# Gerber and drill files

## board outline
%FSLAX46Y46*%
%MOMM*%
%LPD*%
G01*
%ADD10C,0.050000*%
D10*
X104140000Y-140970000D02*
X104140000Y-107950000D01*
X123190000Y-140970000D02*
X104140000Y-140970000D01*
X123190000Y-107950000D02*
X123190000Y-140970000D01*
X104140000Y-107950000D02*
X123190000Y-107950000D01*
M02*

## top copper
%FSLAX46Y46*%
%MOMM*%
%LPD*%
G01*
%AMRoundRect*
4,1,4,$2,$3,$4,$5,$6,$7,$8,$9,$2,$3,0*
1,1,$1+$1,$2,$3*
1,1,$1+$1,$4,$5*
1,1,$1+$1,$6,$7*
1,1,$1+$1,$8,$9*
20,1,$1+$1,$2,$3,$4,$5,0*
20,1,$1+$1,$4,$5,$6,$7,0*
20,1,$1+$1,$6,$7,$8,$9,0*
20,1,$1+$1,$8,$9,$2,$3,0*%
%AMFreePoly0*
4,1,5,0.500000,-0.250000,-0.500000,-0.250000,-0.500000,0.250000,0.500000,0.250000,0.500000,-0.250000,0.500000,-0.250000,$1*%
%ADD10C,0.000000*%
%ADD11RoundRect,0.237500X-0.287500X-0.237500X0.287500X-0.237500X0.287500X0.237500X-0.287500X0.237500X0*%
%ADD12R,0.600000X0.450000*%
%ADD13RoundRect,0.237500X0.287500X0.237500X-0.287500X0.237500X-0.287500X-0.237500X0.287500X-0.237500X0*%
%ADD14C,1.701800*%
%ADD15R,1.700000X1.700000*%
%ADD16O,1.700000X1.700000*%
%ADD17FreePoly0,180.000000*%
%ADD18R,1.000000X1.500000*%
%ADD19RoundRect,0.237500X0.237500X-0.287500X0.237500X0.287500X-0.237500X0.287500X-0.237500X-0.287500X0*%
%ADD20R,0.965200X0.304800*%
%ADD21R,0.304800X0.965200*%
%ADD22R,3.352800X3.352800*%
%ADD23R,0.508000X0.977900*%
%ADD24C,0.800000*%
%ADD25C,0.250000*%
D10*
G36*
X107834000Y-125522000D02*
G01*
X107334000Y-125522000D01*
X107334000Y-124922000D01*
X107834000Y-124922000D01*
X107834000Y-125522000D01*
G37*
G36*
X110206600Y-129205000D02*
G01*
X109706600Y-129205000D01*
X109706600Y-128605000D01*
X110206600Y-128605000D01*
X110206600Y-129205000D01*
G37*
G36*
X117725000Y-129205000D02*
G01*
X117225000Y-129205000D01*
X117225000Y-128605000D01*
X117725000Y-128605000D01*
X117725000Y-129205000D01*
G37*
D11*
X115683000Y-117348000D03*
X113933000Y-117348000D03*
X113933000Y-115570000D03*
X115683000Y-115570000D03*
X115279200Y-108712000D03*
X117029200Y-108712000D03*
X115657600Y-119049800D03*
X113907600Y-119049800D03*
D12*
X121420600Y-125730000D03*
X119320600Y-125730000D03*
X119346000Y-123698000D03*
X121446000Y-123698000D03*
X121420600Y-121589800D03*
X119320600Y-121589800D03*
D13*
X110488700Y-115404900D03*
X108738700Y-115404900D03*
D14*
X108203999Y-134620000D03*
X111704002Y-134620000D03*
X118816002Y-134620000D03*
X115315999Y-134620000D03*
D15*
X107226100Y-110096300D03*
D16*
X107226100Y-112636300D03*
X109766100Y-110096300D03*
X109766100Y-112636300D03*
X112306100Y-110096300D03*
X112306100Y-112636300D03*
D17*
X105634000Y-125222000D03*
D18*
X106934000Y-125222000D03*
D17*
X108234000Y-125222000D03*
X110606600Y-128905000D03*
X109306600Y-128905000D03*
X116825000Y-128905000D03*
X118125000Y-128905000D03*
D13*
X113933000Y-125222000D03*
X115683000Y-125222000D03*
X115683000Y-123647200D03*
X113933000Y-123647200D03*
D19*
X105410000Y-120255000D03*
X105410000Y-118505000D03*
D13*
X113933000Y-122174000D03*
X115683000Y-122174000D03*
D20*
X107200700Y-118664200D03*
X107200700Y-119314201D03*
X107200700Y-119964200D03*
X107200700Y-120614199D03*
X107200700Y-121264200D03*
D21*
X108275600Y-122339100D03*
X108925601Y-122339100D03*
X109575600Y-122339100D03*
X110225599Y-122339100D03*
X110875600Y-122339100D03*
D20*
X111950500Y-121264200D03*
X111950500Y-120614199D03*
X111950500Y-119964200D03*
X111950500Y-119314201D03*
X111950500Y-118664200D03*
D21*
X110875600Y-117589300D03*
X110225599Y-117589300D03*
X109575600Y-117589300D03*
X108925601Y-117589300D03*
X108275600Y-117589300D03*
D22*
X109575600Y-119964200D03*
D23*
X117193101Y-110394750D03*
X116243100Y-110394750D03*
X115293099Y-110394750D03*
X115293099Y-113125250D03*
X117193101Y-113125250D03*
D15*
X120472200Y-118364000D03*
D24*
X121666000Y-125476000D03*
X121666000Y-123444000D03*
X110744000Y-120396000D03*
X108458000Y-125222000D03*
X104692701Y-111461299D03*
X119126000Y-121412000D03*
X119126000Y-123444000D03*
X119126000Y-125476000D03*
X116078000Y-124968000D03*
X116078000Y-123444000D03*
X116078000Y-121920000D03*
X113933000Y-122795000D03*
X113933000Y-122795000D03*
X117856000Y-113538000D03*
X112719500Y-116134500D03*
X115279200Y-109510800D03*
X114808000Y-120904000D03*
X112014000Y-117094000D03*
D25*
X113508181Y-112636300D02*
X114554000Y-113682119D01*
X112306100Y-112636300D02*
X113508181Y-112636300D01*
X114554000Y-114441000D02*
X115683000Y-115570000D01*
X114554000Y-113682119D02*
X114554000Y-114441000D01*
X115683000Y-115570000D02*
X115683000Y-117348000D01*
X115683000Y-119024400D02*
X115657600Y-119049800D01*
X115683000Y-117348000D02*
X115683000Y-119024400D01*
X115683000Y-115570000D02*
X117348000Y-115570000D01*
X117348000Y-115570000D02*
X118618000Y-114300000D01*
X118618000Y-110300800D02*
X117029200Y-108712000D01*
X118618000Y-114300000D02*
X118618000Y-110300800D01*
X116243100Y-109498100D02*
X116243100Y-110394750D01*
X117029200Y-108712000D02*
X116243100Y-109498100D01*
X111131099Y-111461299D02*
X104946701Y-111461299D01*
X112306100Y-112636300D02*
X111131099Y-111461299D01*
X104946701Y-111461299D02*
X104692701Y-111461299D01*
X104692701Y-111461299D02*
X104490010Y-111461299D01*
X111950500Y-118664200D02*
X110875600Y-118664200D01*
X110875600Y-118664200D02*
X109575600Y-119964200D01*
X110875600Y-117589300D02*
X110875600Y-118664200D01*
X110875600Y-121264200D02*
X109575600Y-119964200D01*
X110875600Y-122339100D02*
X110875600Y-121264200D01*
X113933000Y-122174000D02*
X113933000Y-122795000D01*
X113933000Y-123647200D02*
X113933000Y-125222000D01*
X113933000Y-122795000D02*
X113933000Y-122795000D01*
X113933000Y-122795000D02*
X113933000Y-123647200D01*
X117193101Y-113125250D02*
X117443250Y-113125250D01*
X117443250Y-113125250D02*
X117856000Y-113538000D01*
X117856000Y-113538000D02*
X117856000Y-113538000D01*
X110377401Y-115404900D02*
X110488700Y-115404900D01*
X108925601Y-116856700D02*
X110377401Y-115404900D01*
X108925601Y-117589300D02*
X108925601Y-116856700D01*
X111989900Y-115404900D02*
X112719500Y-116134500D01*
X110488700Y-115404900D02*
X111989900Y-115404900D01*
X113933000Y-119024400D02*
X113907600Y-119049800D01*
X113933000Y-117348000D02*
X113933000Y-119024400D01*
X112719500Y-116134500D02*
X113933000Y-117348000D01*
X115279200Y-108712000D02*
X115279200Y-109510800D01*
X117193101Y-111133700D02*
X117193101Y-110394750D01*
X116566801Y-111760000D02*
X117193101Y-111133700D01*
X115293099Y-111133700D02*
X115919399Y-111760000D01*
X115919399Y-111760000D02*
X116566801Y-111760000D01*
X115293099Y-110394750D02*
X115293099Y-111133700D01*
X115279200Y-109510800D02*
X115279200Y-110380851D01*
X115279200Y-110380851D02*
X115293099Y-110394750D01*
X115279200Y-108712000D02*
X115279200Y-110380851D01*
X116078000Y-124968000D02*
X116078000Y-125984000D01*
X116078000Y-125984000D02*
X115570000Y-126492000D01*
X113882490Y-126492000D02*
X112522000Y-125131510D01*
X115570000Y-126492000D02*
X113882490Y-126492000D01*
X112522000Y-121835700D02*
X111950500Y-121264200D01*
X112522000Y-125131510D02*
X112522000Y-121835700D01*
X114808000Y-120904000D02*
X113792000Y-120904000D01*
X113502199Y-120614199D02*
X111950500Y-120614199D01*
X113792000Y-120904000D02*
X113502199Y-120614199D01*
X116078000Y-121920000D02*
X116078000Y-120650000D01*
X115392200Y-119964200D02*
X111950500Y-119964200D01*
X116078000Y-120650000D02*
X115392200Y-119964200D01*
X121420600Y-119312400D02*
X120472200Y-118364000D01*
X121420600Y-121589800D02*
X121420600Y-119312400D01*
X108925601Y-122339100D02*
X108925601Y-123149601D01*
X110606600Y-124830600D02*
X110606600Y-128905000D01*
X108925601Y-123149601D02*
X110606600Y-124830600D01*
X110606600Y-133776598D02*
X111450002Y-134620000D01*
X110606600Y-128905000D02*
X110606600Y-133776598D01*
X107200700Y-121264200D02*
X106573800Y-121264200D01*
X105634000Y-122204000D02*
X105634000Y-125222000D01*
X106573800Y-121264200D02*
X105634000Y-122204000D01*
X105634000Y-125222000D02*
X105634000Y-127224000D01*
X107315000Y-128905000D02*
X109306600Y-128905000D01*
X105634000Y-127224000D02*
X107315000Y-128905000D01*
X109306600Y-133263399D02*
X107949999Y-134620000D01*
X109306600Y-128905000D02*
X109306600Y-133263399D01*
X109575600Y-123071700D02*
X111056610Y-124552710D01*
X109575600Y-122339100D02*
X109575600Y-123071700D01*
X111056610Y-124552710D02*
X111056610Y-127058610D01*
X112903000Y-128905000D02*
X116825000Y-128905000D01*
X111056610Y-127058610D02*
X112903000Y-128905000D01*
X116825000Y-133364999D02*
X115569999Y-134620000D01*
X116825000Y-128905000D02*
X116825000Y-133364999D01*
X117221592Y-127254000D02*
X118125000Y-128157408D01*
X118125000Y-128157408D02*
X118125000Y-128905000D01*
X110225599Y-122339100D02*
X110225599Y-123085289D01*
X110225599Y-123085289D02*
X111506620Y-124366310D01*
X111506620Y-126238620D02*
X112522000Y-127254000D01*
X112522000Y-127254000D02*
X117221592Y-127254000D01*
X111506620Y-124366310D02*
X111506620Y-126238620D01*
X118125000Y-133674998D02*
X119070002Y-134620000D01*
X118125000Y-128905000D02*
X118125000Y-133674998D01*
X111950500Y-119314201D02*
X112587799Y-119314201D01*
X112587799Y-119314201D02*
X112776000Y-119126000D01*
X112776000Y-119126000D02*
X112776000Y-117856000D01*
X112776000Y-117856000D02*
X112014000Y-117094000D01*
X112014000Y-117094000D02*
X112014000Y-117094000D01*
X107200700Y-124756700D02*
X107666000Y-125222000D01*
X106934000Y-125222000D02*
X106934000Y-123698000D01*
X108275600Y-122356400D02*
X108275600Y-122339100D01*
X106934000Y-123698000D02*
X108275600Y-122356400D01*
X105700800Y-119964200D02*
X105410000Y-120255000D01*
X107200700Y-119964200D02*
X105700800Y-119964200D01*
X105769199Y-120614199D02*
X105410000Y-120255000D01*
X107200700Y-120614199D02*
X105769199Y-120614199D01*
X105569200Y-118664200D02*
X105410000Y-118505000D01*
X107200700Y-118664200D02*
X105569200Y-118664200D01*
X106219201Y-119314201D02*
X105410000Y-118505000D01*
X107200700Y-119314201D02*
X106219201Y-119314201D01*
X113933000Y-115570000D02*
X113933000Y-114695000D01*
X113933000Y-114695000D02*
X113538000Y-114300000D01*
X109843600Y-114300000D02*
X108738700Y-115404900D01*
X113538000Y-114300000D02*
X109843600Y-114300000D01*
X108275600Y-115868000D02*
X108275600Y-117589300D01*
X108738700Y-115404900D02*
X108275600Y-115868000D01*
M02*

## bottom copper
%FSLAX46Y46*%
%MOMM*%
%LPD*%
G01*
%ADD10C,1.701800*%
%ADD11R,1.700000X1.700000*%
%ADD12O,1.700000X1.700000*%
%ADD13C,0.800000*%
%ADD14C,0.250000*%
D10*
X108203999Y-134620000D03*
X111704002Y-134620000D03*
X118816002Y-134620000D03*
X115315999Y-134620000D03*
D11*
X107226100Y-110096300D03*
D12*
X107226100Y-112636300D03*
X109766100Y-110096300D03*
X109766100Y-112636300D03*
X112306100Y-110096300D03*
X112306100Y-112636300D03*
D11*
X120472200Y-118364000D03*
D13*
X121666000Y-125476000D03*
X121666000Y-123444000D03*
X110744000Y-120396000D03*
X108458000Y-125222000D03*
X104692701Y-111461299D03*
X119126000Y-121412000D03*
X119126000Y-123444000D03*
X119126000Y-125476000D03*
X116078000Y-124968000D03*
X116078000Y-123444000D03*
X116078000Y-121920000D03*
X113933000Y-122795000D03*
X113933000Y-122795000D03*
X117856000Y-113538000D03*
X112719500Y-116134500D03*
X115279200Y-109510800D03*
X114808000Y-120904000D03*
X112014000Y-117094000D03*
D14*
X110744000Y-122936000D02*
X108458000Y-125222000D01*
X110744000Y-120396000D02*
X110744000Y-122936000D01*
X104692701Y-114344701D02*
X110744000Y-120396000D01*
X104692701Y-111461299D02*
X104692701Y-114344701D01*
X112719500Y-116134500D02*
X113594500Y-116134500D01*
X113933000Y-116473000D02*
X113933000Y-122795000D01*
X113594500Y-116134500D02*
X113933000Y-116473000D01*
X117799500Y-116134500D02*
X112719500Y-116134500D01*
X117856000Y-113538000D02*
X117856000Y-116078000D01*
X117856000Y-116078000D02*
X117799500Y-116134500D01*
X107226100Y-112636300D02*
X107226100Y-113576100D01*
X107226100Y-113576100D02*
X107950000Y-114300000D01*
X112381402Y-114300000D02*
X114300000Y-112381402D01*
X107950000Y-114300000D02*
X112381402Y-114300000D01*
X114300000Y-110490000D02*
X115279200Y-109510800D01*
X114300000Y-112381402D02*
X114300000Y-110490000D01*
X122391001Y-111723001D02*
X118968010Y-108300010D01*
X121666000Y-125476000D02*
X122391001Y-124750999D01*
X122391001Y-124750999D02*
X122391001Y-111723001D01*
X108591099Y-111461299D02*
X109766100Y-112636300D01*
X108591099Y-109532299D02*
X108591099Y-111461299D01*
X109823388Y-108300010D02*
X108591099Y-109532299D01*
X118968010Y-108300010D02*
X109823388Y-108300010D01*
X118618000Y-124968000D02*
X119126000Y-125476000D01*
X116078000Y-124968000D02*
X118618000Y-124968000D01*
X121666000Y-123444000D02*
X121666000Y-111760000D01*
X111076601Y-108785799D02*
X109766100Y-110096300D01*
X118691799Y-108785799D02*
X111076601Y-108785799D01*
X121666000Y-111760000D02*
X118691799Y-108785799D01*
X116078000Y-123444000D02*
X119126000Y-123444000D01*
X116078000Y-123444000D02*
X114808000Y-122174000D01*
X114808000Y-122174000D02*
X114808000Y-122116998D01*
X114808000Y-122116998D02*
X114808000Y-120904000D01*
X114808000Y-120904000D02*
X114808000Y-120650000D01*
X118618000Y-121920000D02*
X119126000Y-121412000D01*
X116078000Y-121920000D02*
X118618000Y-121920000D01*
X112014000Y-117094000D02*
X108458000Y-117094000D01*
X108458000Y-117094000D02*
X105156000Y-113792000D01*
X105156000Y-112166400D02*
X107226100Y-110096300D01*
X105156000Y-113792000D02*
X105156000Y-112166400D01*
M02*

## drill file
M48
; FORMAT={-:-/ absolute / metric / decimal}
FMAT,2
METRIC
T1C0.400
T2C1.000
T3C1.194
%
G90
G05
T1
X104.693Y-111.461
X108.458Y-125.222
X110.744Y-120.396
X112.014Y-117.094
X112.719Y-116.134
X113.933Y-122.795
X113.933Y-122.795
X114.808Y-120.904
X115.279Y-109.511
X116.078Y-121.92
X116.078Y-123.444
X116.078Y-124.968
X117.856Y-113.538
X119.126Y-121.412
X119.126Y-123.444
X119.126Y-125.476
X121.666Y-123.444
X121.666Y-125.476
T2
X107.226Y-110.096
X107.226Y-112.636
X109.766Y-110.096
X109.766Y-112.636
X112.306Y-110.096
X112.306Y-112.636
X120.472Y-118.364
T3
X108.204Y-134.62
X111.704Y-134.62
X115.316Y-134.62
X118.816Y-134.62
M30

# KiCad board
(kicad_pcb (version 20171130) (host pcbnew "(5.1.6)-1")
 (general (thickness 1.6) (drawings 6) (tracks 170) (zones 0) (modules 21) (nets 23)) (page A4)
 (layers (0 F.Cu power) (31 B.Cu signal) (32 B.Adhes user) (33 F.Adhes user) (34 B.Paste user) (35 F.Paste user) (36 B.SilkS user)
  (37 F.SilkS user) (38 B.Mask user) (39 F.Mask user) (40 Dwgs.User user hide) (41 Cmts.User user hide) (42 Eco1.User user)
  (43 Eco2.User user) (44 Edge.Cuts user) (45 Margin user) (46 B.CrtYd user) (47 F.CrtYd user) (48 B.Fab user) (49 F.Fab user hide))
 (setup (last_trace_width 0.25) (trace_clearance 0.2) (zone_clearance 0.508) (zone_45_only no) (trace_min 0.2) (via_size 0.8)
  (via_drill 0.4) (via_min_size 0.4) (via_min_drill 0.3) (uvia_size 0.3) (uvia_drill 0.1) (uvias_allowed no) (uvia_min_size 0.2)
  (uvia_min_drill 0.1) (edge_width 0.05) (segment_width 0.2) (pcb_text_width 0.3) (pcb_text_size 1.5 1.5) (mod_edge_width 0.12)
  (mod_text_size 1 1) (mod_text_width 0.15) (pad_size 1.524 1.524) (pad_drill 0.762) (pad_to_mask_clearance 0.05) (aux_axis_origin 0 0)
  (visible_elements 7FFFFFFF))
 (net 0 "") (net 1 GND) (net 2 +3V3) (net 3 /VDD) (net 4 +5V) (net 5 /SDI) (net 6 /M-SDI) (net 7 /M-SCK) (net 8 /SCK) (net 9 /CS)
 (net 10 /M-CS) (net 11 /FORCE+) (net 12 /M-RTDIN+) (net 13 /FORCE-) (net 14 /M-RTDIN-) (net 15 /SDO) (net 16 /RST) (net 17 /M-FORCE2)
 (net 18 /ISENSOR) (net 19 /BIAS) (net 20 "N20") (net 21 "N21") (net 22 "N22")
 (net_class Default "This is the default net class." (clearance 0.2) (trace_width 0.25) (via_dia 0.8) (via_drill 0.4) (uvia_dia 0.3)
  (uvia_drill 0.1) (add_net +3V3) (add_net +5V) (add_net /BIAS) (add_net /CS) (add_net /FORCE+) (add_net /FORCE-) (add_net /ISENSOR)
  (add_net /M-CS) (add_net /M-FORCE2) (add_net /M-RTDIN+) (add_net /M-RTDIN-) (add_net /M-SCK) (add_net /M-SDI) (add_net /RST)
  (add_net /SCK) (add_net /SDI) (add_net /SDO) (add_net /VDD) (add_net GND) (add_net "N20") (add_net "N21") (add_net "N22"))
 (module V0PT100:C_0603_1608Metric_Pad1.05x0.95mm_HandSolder (layer F.Cu) (at 114.808 117.348)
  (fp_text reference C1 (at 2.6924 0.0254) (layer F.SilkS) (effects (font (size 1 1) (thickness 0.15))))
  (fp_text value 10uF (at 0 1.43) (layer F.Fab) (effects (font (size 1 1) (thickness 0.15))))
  (pad 2 smd roundrect (at 0.875 0) (size 1.05 0.95) (layers F.Cu F.Paste F.Mask) (roundrect_rratio 0.25) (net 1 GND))
  (pad 1 smd roundrect (at -0.875 0) (size 1.05 0.95) (layers F.Cu F.Paste F.Mask) (roundrect_rratio 0.25) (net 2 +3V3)))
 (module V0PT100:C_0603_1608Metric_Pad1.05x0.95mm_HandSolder (layer F.Cu) (at 114.808 115.57)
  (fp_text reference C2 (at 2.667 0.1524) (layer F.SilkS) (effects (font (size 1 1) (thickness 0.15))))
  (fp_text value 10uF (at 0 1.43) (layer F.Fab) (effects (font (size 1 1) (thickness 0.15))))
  (pad 1 smd roundrect (at -0.875 0) (size 1.05 0.95) (layers F.Cu F.Paste F.Mask) (roundrect_rratio 0.25) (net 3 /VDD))
  (pad 2 smd roundrect (at 0.875 0) (size 1.05 0.95) (layers F.Cu F.Paste F.Mask) (roundrect_rratio 0.25) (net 1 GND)))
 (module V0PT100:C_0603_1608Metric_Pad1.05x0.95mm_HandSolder (layer F.Cu) (at 116.1542 108.712)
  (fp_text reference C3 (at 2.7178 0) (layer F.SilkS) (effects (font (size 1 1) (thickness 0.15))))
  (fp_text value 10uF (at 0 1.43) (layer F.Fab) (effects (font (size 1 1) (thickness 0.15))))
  (pad 1 smd roundrect (at -0.875 0) (size 1.05 0.95) (layers F.Cu F.Paste F.Mask) (roundrect_rratio 0.25) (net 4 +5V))
  (pad 2 smd roundrect (at 0.875 0) (size 1.05 0.95) (layers F.Cu F.Paste F.Mask) (roundrect_rratio 0.25) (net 1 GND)))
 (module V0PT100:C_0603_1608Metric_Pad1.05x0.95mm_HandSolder (layer F.Cu) (at 114.7826 119.0498)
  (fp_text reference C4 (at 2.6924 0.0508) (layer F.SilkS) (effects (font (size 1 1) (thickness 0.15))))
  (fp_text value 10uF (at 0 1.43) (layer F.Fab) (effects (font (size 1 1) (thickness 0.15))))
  (pad 2 smd roundrect (at 0.875 0) (size 1.05 0.95) (layers F.Cu F.Paste F.Mask) (roundrect_rratio 0.25) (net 1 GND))
  (pad 1 smd roundrect (at -0.875 0) (size 1.05 0.95) (layers F.Cu F.Paste F.Mask) (roundrect_rratio 0.25) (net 2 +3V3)))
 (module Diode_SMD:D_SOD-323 (layer F.Cu) (at 120.3706 125.73 180)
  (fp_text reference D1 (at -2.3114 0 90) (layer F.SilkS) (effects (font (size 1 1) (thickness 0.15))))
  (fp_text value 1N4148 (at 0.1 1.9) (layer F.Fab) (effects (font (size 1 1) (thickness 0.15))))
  (pad 1 smd rect (at -1.05 0 180) (size 0.6 0.45) (layers F.Cu F.Paste F.Mask) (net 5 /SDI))
  (pad 2 smd rect (at 1.05 0 180) (size 0.6 0.45) (layers F.Cu F.Paste F.Mask) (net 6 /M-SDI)))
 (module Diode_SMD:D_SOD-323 (layer F.Cu) (at 120.396 123.698 180)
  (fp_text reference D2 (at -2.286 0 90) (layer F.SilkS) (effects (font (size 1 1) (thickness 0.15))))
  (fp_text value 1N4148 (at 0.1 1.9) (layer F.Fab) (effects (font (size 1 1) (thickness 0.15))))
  (pad 2 smd rect (at 1.05 0 180) (size 0.6 0.45) (layers F.Cu F.Paste F.Mask) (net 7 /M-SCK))
  (pad 1 smd rect (at -1.05 0 180) (size 0.6 0.45) (layers F.Cu F.Paste F.Mask) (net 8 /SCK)))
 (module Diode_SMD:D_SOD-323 (layer F.Cu) (at 120.3706 121.5898 180)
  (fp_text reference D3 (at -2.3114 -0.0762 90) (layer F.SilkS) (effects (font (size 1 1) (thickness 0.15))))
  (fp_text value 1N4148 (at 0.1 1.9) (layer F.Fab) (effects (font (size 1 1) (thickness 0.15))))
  (pad 1 smd rect (at -1.05 0 180) (size 0.6 0.45) (layers F.Cu F.Paste F.Mask) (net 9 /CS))
  (pad 2 smd rect (at 1.05 0 180) (size 0.6 0.45) (layers F.Cu F.Paste F.Mask) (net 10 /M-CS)))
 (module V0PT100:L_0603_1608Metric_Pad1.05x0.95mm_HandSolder (layer F.Cu) (at 109.6137 115.4049 180)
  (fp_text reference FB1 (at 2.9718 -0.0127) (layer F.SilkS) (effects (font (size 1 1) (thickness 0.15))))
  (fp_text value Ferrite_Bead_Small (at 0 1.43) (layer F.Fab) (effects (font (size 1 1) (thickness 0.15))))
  (pad 1 smd roundrect (at -0.875 0 180) (size 1.05 0.95) (layers F.Cu F.Paste F.Mask) (roundrect_rratio 0.25) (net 2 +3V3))
  (pad 2 smd roundrect (at 0.875 0 180) (size 1.05 0.95) (layers F.Cu F.Paste F.Mask) (roundrect_rratio 0.25) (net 3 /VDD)))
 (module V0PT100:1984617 (layer F.Cu) (at 108.204 134.62)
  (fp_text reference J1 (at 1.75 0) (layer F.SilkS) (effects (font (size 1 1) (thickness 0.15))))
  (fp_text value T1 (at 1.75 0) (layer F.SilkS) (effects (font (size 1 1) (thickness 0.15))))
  (pad 1 thru_hole circle (at -0.000001 0) (size 1.7018 1.7018) (drill 1.1938) (layers *.Cu *.Mask) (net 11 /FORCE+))
  (pad 2 thru_hole circle (at 3.500002 0) (size 1.7018 1.7018) (drill 1.1938) (layers *.Cu *.Mask) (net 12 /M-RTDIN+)))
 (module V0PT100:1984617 (layer F.Cu) (at 115.316 134.62)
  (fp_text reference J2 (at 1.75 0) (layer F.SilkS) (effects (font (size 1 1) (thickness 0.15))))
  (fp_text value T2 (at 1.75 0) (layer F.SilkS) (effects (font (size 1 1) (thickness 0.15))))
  (pad 2 thru_hole circle (at 3.500002 0) (size 1.7018 1.7018) (drill 1.1938) (layers *.Cu *.Mask) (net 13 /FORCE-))
  (pad 1 thru_hole circle (at -0.000001 0) (size 1.7018 1.7018) (drill 1.1938) (layers *.Cu *.Mask) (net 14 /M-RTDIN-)))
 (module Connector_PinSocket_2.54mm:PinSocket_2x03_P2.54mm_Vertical (layer F.Cu) (at 107.2261 110.0963 90)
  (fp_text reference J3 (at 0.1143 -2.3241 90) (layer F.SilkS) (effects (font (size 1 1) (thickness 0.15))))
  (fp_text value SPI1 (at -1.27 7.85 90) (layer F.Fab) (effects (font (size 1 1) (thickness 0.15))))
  (pad 1 thru_hole rect (at 0 0 90) (size 1.7 1.7) (drill 1) (layers *.Cu *.Mask) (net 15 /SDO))
  (pad 2 thru_hole oval (at -2.54 0 90) (size 1.7 1.7) (drill 1) (layers *.Cu *.Mask) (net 4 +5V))
  (pad 3 thru_hole oval (at 0 2.54 90) (size 1.7 1.7) (drill 1) (layers *.Cu *.Mask) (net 8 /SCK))
  (pad 4 thru_hole oval (at -2.54 2.54 90) (size 1.7 1.7) (drill 1) (layers *.Cu *.Mask) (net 5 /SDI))
  (pad 5 thru_hole oval (at 0 5.08 90) (size 1.7 1.7) (drill 1) (layers *.Cu *.Mask) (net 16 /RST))
  (pad 6 thru_hole oval (at -2.54 5.08 90) (size 1.7 1.7) (drill 1) (layers *.Cu *.Mask) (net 1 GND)))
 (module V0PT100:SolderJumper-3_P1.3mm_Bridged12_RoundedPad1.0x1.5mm (layer F.Cu) (at 106.934 125.222 180)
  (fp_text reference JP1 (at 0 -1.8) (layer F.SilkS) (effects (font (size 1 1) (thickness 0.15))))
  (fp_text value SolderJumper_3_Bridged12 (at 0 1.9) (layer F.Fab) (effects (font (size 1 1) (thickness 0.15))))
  (fp_poly (pts (xy -0.9 -0.3) (xy -0.4 -0.3) (xy -0.4 0.3) (xy -0.9 0.3)) (layer F.Cu) (width 0))
  (pad 3 smd custom (at 1.3 0 180) (size 1 0.5) (layers F.Cu F.Mask) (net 11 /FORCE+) (zone_connect 2)
   (options (clearance outline) (anchor rect)) (primitives))
  (pad 2 smd rect (at 0 0 180) (size 1 1.5) (layers F.Cu F.Mask) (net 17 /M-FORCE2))
  (pad 1 smd custom (at -1.3 0 180) (size 1 0.5) (layers F.Cu F.Mask) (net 1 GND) (zone_connect 2)
   (options (clearance outline) (anchor rect)) (primitives)))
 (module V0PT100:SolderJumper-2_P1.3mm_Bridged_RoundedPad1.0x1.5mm (layer F.Cu) (at 109.9566 128.905 180)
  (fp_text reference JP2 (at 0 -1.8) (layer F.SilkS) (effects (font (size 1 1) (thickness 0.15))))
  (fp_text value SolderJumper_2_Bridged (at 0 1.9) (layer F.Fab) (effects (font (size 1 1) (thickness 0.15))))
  (fp_poly (pts (xy 0.25 -0.3) (xy -0.25 -0.3) (xy -0.25 0.3) (xy 0.25 0.3)) (layer F.Cu) (width 0))
  (pad 1 smd custom (at -0.65 0 180) (size 1 0.5) (layers F.Cu F.Mask) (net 12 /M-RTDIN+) (zone_connect 2)
   (options (clearance outline) (anchor rect)) (primitives))
  (pad 2 smd custom (at 0.65 0 180) (size 1 0.5) (layers F.Cu F.Mask) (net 11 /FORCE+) (zone_connect 2)
   (options (clearance outline) (anchor rect)) (primitives)))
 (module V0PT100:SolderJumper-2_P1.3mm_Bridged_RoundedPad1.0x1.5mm (layer F.Cu) (at 117.475 128.905 180)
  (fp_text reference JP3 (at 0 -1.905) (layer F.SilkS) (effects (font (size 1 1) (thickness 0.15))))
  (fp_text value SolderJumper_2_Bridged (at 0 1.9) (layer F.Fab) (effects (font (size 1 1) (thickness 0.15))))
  (fp_poly (pts (xy 0.25 -0.3) (xy -0.25 -0.3) (xy -0.25 0.3) (xy 0.25 0.3)) (layer F.Cu) (width 0))
  (pad 2 smd custom (at 0.65 0 180) (size 1 0.5) (layers F.Cu F.Mask) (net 14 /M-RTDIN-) (zone_connect 2)
   (options (clearance outline) (anchor rect)) (primitives))
  (pad 1 smd custom (at -0.65 0 180) (size 1 0.5) (layers F.Cu F.Mask) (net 13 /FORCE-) (zone_connect 2)
   (options (clearance outline) (anchor rect)) (primitives)))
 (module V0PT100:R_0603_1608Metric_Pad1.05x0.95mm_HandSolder (layer F.Cu) (at 114.808 125.222 180)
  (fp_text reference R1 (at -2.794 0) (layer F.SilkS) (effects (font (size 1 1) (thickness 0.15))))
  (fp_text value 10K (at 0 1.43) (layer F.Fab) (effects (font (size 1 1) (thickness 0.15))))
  (pad 2 smd roundrect (at 0.875 0 180) (size 1.05 0.95) (layers F.Cu F.Paste F.Mask) (roundrect_rratio 0.25) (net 2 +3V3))
  (pad 1 smd roundrect (at -0.875 0 180) (size 1.05 0.95) (layers F.Cu F.Paste F.Mask) (roundrect_rratio 0.25) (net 6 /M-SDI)))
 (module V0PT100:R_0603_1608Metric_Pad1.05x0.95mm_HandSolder (layer F.Cu) (at 114.808 123.6472 180)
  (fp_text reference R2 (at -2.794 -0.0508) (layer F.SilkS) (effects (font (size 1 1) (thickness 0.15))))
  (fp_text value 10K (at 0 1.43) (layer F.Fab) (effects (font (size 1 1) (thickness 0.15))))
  (pad 1 smd roundrect (at -0.875 0 180) (size 1.05 0.95) (layers F.Cu F.Paste F.Mask) (roundrect_rratio 0.25) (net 7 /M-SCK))
  (pad 2 smd roundrect (at 0.875 0 180) (size 1.05 0.95) (layers F.Cu F.Paste F.Mask) (roundrect_rratio 0.25) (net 2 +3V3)))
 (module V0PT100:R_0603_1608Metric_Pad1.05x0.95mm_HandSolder (layer F.Cu) (at 105.41 119.38 90)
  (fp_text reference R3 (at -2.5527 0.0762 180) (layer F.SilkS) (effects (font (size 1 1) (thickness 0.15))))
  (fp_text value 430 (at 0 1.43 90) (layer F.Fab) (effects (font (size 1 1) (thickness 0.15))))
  (pad 1 smd roundrect (at -0.875 0 90) (size 1.05 0.95) (layers F.Cu F.Paste F.Mask) (roundrect_rratio 0.25) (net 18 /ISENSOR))
  (pad 2 smd roundrect (at 0.875 0 90) (size 1.05 0.95) (layers F.Cu F.Paste F.Mask) (roundrect_rratio 0.25) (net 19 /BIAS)))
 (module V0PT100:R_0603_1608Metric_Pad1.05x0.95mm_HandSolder (layer F.Cu) (at 114.808 122.174 180)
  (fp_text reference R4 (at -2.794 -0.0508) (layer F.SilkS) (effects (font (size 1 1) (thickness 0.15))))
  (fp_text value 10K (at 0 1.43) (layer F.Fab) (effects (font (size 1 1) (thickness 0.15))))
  (pad 2 smd roundrect (at 0.875 0 180) (size 1.05 0.95) (layers F.Cu F.Paste F.Mask) (roundrect_rratio 0.25) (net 2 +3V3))
  (pad 1 smd roundrect (at -0.875 0 180) (size 1.05 0.95) (layers F.Cu F.Paste F.Mask) (roundrect_rratio 0.25) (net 10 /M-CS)))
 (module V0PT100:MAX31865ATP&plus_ (layer F.Cu) (at 109.5756 119.9642)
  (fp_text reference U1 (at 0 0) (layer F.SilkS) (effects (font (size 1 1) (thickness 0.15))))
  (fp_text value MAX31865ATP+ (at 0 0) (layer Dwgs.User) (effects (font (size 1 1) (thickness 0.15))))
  (pad 1 smd rect (at -2.3749 -1.3 90) (size 0.3048 0.9652) (layers F.Cu F.Paste F.Mask) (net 19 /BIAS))
  (pad 2 smd rect (at -2.3749 -0.649999 90) (size 0.3048 0.9652) (layers F.Cu F.Paste F.Mask) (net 19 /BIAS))
  (pad 3 smd rect (at -2.3749 0 90) (size 0.3048 0.9652) (layers F.Cu F.Paste F.Mask) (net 18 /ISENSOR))
  (pad 4 smd rect (at -2.3749 0.649999 90) (size 0.3048 0.9652) (layers F.Cu F.Paste F.Mask) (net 18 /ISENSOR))
  (pad 5 smd rect (at -2.3749 1.3 90) (size 0.3048 0.9652) (layers F.Cu F.Paste F.Mask) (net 11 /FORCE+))
  (pad 6 smd rect (at -1.3 2.3749) (size 0.3048 0.9652) (layers F.Cu F.Paste F.Mask) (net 17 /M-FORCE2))
  (pad 7 smd rect (at -0.649999 2.3749) (size 0.3048 0.9652) (layers F.Cu F.Paste F.Mask) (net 12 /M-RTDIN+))
  (pad 8 smd rect (at 0 2.3749) (size 0.3048 0.9652) (layers F.Cu F.Paste F.Mask) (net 14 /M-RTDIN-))
  (pad 9 smd rect (at 0.649999 2.3749) (size 0.3048 0.9652) (layers F.Cu F.Paste F.Mask) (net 13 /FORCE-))
  (pad 10 smd rect (at 1.3 2.3749) (size 0.3048 0.9652) (layers F.Cu F.Paste F.Mask) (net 1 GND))
  (pad 11 smd rect (at 2.3749 1.3 90) (size 0.3048 0.9652) (layers F.Cu F.Paste F.Mask) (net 6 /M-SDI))
  (pad 12 smd rect (at 2.3749 0.649999 90) (size 0.3048 0.9652) (layers F.Cu F.Paste F.Mask) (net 7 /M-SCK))
  (pad 13 smd rect (at 2.3749 0 90) (size 0.3048 0.9652) (layers F.Cu F.Paste F.Mask) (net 10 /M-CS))
  (pad 14 smd rect (at 2.3749 -0.649999 90) (size 0.3048 0.9652) (layers F.Cu F.Paste F.Mask) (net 15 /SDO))
  (pad 15 smd rect (at 2.3749 -1.3 90) (size 0.3048 0.9652) (layers F.Cu F.Paste F.Mask) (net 1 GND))
  (pad 16 smd rect (at 1.3 -2.3749) (size 0.3048 0.9652) (layers F.Cu F.Paste F.Mask) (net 1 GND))
  (pad 17 smd rect (at 0.649999 -2.3749) (size 0.3048 0.9652) (layers F.Cu F.Paste F.Mask) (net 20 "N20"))
  (pad 18 smd rect (at 0 -2.3749) (size 0.3048 0.9652) (layers F.Cu F.Paste F.Mask) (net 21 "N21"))
  (pad 19 smd rect (at -0.649999 -2.3749) (size 0.3048 0.9652) (layers F.Cu F.Paste F.Mask) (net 2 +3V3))
  (pad 20 smd rect (at -1.3 -2.3749) (size 0.3048 0.9652) (layers F.Cu F.Paste F.Mask) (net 3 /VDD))
  (pad 21 smd rect (at 0 0) (size 3.3528 3.3528) (layers F.Cu F.Paste F.Mask) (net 1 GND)))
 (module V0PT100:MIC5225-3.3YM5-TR (layer F.Cu) (at 116.2431 111.76 270)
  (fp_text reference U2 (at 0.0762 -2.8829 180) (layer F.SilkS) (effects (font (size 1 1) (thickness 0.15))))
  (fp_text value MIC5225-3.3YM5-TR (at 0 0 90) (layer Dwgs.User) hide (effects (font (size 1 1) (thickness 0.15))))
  (pad 1 smd rect (at -1.36525 -0.950001 270) (size 0.9779 0.508) (layers F.Cu F.Paste F.Mask) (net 4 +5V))
  (pad 2 smd rect (at -1.36525 0 270) (size 0.9779 0.508) (layers F.Cu F.Paste F.Mask) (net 1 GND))
  (pad 3 smd rect (at -1.36525 0.950001 270) (size 0.9779 0.508) (layers F.Cu F.Paste F.Mask) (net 4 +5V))
  (pad 4 smd rect (at 1.36525 0.950001 270) (size 0.9779 0.508) (layers F.Cu F.Paste F.Mask) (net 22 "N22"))
  (pad 5 smd rect (at 1.36525 -0.950001 270) (size 0.9779 0.508) (layers F.Cu F.Paste F.Mask) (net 2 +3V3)))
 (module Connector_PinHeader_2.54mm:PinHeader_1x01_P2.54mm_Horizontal (layer F.Cu) (at 120.4722 118.364 90)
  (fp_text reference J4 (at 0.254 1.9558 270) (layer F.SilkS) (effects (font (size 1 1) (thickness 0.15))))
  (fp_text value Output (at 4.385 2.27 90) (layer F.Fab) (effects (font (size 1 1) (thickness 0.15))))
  (pad 1 thru_hole rect (at 0 0 90) (size 1.7 1.7) (drill 1) (layers *.Cu *.Mask) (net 9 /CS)))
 (gr_line (start 104.14 140.97) (end 104.14 107.95) (layer Edge.Cuts) (width 0.05))
 (gr_line (start 123.19 140.97) (end 104.14 140.97) (layer Edge.Cuts) (width 0.05))
 (gr_line (start 123.19 107.95) (end 123.19 140.97) (layer Edge.Cuts) (width 0.05))
 (gr_line (start 104.14 107.95) (end 123.19 107.95) (layer Edge.Cuts) (width 0.05))
 (via (at 121.666 125.476) (size 0.8) (drill 0.4) (layers F.Cu B.Cu) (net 5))
 (via (at 121.666 123.444) (size 0.8) (drill 0.4) (layers F.Cu B.Cu) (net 8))
 (via (at 110.744 120.396) (size 0.8) (drill 0.4) (layers F.Cu B.Cu) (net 1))
 (via (at 108.458 125.222) (size 0.8) (drill 0.4) (layers F.Cu B.Cu) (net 1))
 (segment (start 110.744 122.936) (end 108.458 125.222) (width 0.25) (layer B.Cu) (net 1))
 (segment (start 110.744 120.396) (end 110.744 122.936) (width 0.25) (layer B.Cu) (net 1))
 (segment (start 113.508181 112.6363) (end 114.554 113.682119) (width 0.25) (layer F.Cu) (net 1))
 (segment (start 112.3061 112.6363) (end 113.508181 112.6363) (width 0.25) (layer F.Cu) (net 1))
 (segment (start 114.554 114.441) (end 115.683 115.57) (width 0.25) (layer F.Cu) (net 1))
 (segment (start 114.554 113.682119) (end 114.554 114.441) (width 0.25) (layer F.Cu) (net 1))
 (segment (start 115.683 115.57) (end 115.683 117.348) (width 0.25) (layer F.Cu) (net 1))
 (segment (start 115.683 119.0244) (end 115.6576 119.0498) (width 0.25) (layer F.Cu) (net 1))
 (segment (start 115.683 117.348) (end 115.683 119.0244) (width 0.25) (layer F.Cu) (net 1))
 (segment (start 115.683 115.57) (end 117.348 115.57) (width 0.25) (layer F.Cu) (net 1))
 (segment (start 117.348 115.57) (end 118.618 114.3) (width 0.25) (layer F.Cu) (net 1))
 (segment (start 118.618 110.3008) (end 117.0292 108.712) (width 0.25) (layer F.Cu) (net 1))
 (segment (start 118.618 114.3) (end 118.618 110.3008) (width 0.25) (layer F.Cu) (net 1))
 (segment (start 116.2431 109.4981) (end 116.2431 110.39475) (width 0.25) (layer F.Cu) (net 1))
 (segment (start 117.0292 108.712) (end 116.2431 109.4981) (width 0.25) (layer F.Cu) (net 1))
 (segment (start 111.131099 111.461299) (end 104.946701 111.461299) (width 0.25) (layer F.Cu) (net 1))
 (segment (start 112.3061 112.6363) (end 111.131099 111.461299) (width 0.25) (layer F.Cu) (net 1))
 (segment (start 104.946701 111.461299) (end 104.692701 111.461299) (width 0.25) (layer F.Cu) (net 1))
 (segment (start 104.692701 111.461299) (end 104.49001 111.461299) (width 0.25) (layer F.Cu) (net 1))
 (via (at 104.692701 111.461299) (size 0.8) (drill 0.4) (layers F.Cu B.Cu) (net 1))
 (segment (start 104.692701 114.344701) (end 110.744 120.396) (width 0.25) (layer B.Cu) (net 1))
 (segment (start 104.692701 111.461299) (end 104.692701 114.344701) (width 0.25) (layer B.Cu) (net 1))
 (segment (start 111.9505 118.6642) (end 110.8756 118.6642) (width 0.25) (layer F.Cu) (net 1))
 (segment (start 110.8756 118.6642) (end 109.5756 119.9642) (width 0.25) (layer F.Cu) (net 1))
 (segment (start 110.8756 117.5893) (end 110.8756 118.6642) (width 0.25) (layer F.Cu) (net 1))
 (segment (start 110.8756 121.2642) (end 109.5756 119.9642) (width 0.25) (layer F.Cu) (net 1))
 (segment (start 110.8756 122.3391) (end 110.8756 121.2642) (width 0.25) (layer F.Cu) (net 1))
 (via (at 119.126 121.412) (size 0.8) (drill 0.4) (layers F.Cu B.Cu) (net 10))
 (via (at 119.126 123.444) (size 0.8) (drill 0.4) (layers F.Cu B.Cu) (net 7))
 (via (at 119.126 125.476) (size 0.8) (drill 0.4) (layers F.Cu B.Cu) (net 6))
 (via (at 116.078 124.968) (size 0.8) (drill 0.4) (layers F.Cu B.Cu) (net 6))
 (via (at 116.078 123.444) (size 0.8) (drill 0.4) (layers F.Cu B.Cu) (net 7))
 (via (at 116.078 121.92) (size 0.8) (drill 0.4) (layers F.Cu B.Cu) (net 10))
 (segment (start 113.933 122.174) (end 113.933 122.795) (width 0.25) (layer F.Cu) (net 2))
 (segment (start 113.933 123.6472) (end 113.933 125.222) (width 0.25) (layer F.Cu) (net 2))
 (segment (start 113.933 122.795) (end 113.933 122.795) (width 0.25) (layer F.Cu) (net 2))
 (via (at 113.933 122.795) (size 0.8) (drill 0.4) (layers F.Cu B.Cu) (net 2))
 (segment (start 113.933 122.795) (end 113.933 123.6472) (width 0.25) (layer F.Cu) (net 2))
 (via (at 113.933 122.795) (size 0.8) (drill 0.4) (layers F.Cu B.Cu) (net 2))
 (segment (start 117.193101 113.12525) (end 117.44325 113.12525) (width 0.25) (layer F.Cu) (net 2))
 (segment (start 117.44325 113.12525) (end 117.856 113.538) (width 0.25) (layer F.Cu) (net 2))
 (segment (start 117.856 113.538) (end 117.856 113.538) (width 0.25) (layer F.Cu) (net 2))
 (via (at 117.856 113.538) (size 0.8) (drill 0.4) (layers F.Cu B.Cu) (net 2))
 (segment (start 110.377401 115.4049) (end 110.4887 115.4049) (width 0.25) (layer F.Cu) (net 2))
 (segment (start 108.925601 116.8567) (end 110.377401 115.4049) (width 0.25) (layer F.Cu) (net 2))
 (segment (start 108.925601 117.5893) (end 108.925601 116.8567) (width 0.25) (layer F.Cu) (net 2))
 (segment (start 111.9899 115.4049) (end 112.7195 116.1345) (width 0.25) (layer F.Cu) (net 2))
 (segment (start 110.4887 115.4049) (end 111.9899 115.4049) (width 0.25) (layer F.Cu) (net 2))
 (segment (start 113.933 119.0244) (end 113.9076 119.0498) (width 0.25) (layer F.Cu) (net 2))
 (segment (start 113.933 117.348) (end 113.933 119.0244) (width 0.25) (layer F.Cu) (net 2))
 (segment (start 112.7195 116.1345) (end 113.933 117.348) (width 0.25) (layer F.Cu) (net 2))
 (via (at 112.7195 116.1345) (size 0.8) (drill 0.4) (layers F.Cu B.Cu) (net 2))
 (segment (start 112.7195 116.1345) (end 113.5945 116.1345) (width 0.25) (layer B.Cu) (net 2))
 (segment (start 113.933 116.473) (end 113.933 122.795) (width 0.25) (layer B.Cu) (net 2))
 (segment (start 113.5945 116.1345) (end 113.933 116.473) (width 0.25) (layer B.Cu) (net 2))
 (segment (start 117.7995 116.1345) (end 112.7195 116.1345) (width 0.25) (layer B.Cu) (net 2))
 (segment (start 117.856 113.538) (end 117.856 116.078) (width 0.25) (layer B.Cu) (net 2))
 (segment (start 117.856 116.078) (end 117.7995 116.1345) (width 0.25) (layer B.Cu) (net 2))
 (segment (start 107.2261 112.6363) (end 107.2261 113.5761) (width 0.25) (layer B.Cu) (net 4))
 (segment (start 107.2261 113.5761) (end 107.95 114.3) (width 0.25) (layer B.Cu) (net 4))
 (segment (start 112.381402 114.3) (end 114.3 112.381402) (width 0.25) (layer B.Cu) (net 4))
 (segment (start 107.95 114.3) (end 112.381402 114.3) (width 0.25) (layer B.Cu) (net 4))
 (segment (start 115.2792 108.712) (end 115.2792 109.5108) (width 0.25) (layer F.Cu) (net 4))
 (segment (start 117.193101 111.1337) (end 117.193101 110.39475) (width 0.25) (layer F.Cu) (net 4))
 (segment (start 116.566801 111.76) (end 117.193101 111.1337) (width 0.25) (layer F.Cu) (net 4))
 (segment (start 115.293099 111.1337) (end 115.919399 111.76) (width 0.25) (layer F.Cu) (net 4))
 (segment (start 115.919399 111.76) (end 116.566801 111.76) (width 0.25) (layer F.Cu) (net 4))
 (segment (start 115.293099 110.39475) (end 115.293099 111.1337) (width 0.25) (layer F.Cu) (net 4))
 (segment (start 115.2792 109.5108) (end 115.2792 110.380851) (width 0.25) (layer F.Cu) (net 4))
 (via (at 115.2792 109.5108) (size 0.8) (drill 0.4) (layers F.Cu B.Cu) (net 4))
 (segment (start 114.3 110.49) (end 115.2792 109.5108) (width 0.25) (layer B.Cu) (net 4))
 (segment (start 114.3 112.381402) (end 114.3 110.49) (width 0.25) (layer B.Cu) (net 4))
 (segment (start 115.2792 110.380851) (end 115.293099 110.39475) (width 0.25) (layer F.Cu) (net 4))
 (segment (start 115.2792 108.712) (end 115.2792 110.380851) (width 0.25) (layer F.Cu) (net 4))
 (segment (start 122.391001 111.723001) (end 118.96801 108.30001) (width 0.25) (layer B.Cu) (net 5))
 (segment (start 121.666 125.476) (end 122.391001 124.750999) (width 0.25) (layer B.Cu) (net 5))
 (segment (start 122.391001 124.750999) (end 122.391001 111.723001) (width 0.25) (layer B.Cu) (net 5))
 (segment (start 108.591099 111.461299) (end 109.7661 112.6363) (width 0.25) (layer B.Cu) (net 5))
 (segment (start 108.591099 109.532299) (end 108.591099 111.461299) (width 0.25) (layer B.Cu) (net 5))
 (segment (start 109.823388 108.30001) (end 108.591099 109.532299) (width 0.25) (layer B.Cu) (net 5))
 (segment (start 118.96801 108.30001) (end 109.823388 108.30001) (width 0.25) (layer B.Cu) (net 5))
 (segment (start 118.618 124.968) (end 119.126 125.476) (width 0.25) (layer B.Cu) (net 6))
 (segment (start 116.078 124.968) (end 118.618 124.968) (width 0.25) (layer B.Cu) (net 6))
 (segment (start 116.078 124.968) (end 116.078 125.984) (width 0.25) (layer F.Cu) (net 6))
 (segment (start 116.078 125.984) (end 115.57 126.492) (width 0.25) (layer F.Cu) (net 6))
 (segment (start 113.88249 126.492) (end 112.522 125.13151) (width 0.25) (layer F.Cu) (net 6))
 (segment (start 115.57 126.492) (end 113.88249 126.492) (width 0.25) (layer F.Cu) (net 6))
 (segment (start 112.522 121.8357) (end 111.9505 121.2642) (width 0.25) (layer F.Cu) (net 6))
 (segment (start 112.522 125.13151) (end 112.522 121.8357) (width 0.25) (layer F.Cu) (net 6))
 (segment (start 121.666 123.444) (end 121.666 111.76) (width 0.25) (layer B.Cu) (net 8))
 (segment (start 111.076601 108.785799) (end 109.7661 110.0963) (width 0.25) (layer B.Cu) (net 8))
 (segment (start 118.691799 108.785799) (end 111.076601 108.785799) (width 0.25) (layer B.Cu) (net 8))
 (segment (start 121.666 111.76) (end 118.691799 108.785799) (width 0.25) (layer B.Cu) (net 8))
 (segment (start 116.078 123.444) (end 119.126 123.444) (width 0.25) (layer B.Cu) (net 7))
 (segment (start 116.078 123.444) (end 114.808 122.174) (width 0.25) (layer B.Cu) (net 7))
 (segment (start 114.808 122.174) (end 114.808 122.116998) (width 0.25) (layer B.Cu) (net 7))
 (segment (start 114.808 122.116998) (end 114.808 120.904) (width 0.25) (layer B.Cu) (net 7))
 (segment (start 114.808 120.904) (end 114.808 120.65) (width 0.25) (layer B.Cu) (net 7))
 (via (at 114.808 120.904) (size 0.8) (drill 0.4) (layers F.Cu B.Cu) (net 7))
 (segment (start 114.808 120.904) (end 113.792 120.904) (width 0.25) (layer F.Cu) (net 7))
 (segment (start 113.502199 120.614199) (end 111.9505 120.614199) (width 0.25) (layer F.Cu) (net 7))
 (segment (start 113.792 120.904) (end 113.502199 120.614199) (width 0.25) (layer F.Cu) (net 7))
 (segment (start 118.618 121.92) (end 119.126 121.412) (width 0.25) (layer B.Cu) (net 10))
 (segment (start 116.078 121.92) (end 118.618 121.92) (width 0.25) (layer B.Cu) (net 10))
 (segment (start 116.078 121.92) (end 116.078 120.65) (width 0.25) (layer F.Cu) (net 10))
 (segment (start 115.3922 119.9642) (end 111.9505 119.9642) (width 0.25) (layer F.Cu) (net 10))
 (segment (start 116.078 120.65) (end 115.3922 119.9642) (width 0.25) (layer F.Cu) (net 10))
 (segment (start 121.4206 119.3124) (end 120.4722 118.364) (width 0.25) (layer F.Cu) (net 9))
 (segment (start 121.4206 121.5898) (end 121.4206 119.3124) (width 0.25) (layer F.Cu) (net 9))
 (segment (start 108.925601 122.3391) (end 108.925601 123.149601) (width 0.25) (layer F.Cu) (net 12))
 (segment (start 110.6066 124.8306) (end 110.6066 128.905) (width 0.25) (layer F.Cu) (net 12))
 (segment (start 108.925601 123.149601) (end 110.6066 124.8306) (width 0.25) (layer F.Cu) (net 12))
 (segment (start 110.6066 133.776598) (end 111.450002 134.62) (width 0.25) (layer F.Cu) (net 12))
 (segment (start 110.6066 128.905) (end 110.6066 133.776598) (width 0.25) (layer F.Cu) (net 12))
 (segment (start 107.2007 121.2642) (end 106.5738 121.2642) (width 0.25) (layer F.Cu) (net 11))
 (segment (start 105.634 122.204) (end 105.634 125.222) (width 0.25) (layer F.Cu) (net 11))
 (segment (start 106.5738 121.2642) (end 105.634 122.204) (width 0.25) (layer F.Cu) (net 11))
 (segment (start 105.634 125.222) (end 105.634 127.224) (width 0.25) (layer F.Cu) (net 11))
 (segment (start 107.315 128.905) (end 109.3066 128.905) (width 0.25) (layer F.Cu) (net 11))
 (segment (start 105.634 127.224) (end 107.315 128.905) (width 0.25) (layer F.Cu) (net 11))
 (segment (start 109.3066 133.263399) (end 107.949999 134.62) (width 0.25) (layer F.Cu) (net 11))
 (segment (start 109.3066 128.905) (end 109.3066 133.263399) (width 0.25) (layer F.Cu) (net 11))
 (segment (start 109.5756 123.0717) (end 111.05661 124.55271) (width 0.25) (layer F.Cu) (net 14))
 (segment (start 109.5756 122.3391) (end 109.5756 123.0717) (width 0.25) (layer F.Cu) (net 14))
 (segment (start 111.05661 124.55271) (end 111.05661 127.05861) (width 0.25) (layer F.Cu) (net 14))
 (segment (start 112.903 128.905) (end 116.825 128.905) (width 0.25) (layer F.Cu) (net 14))
 (segment (start 111.05661 127.05861) (end 112.903 128.905) (width 0.25) (layer F.Cu) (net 14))
 (segment (start 116.825 133.364999) (end 115.569999 134.62) (width 0.25) (layer F.Cu) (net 14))
 (segment (start 116.825 128.905) (end 116.825 133.364999) (width 0.25) (layer F.Cu) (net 14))
 (segment (start 117.221592 127.254) (end 118.125 128.157408) (width 0.25) (layer F.Cu) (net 13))
 (segment (start 118.125 128.157408) (end 118.125 128.905) (width 0.25) (layer F.Cu) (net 13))
 (segment (start 110.225599 122.3391) (end 110.225599 123.085289) (width 0.25) (layer F.Cu) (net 13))
 (segment (start 110.225599 123.085289) (end 111.50662 124.36631) (width 0.25) (layer F.Cu) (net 13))
 (segment (start 111.50662 126.23862) (end 112.522 127.254) (width 0.25) (layer F.Cu) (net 13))
 (segment (start 112.522 127.254) (end 117.221592 127.254) (width 0.25) (layer F.Cu) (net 13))
 (segment (start 111.50662 124.36631) (end 111.50662 126.23862) (width 0.25) (layer F.Cu) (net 13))
 (segment (start 118.125 133.674998) (end 119.070002 134.62) (width 0.25) (layer F.Cu) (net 13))
 (segment (start 118.125 128.905) (end 118.125 133.674998) (width 0.25) (layer F.Cu) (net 13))
 (segment (start 111.9505 119.314201) (end 112.587799 119.314201) (width 0.25) (layer F.Cu) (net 15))
 (segment (start 112.587799 119.314201) (end 112.776 119.126) (width 0.25) (layer F.Cu) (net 15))
 (segment (start 112.776 119.126) (end 112.776 117.856) (width 0.25) (layer F.Cu) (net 15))
 (segment (start 112.776 117.856) (end 112.014 117.094) (width 0.25) (layer F.Cu) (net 15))
 (segment (start 112.014 117.094) (end 112.014 117.094) (width 0.25) (layer F.Cu) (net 15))
 (via (at 112.014 117.094) (size 0.8) (drill 0.4) (layers F.Cu B.Cu) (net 15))
 (segment (start 112.014 117.094) (end 108.458 117.094) (width 0.25) (layer B.Cu) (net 15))
 (segment (start 108.458 117.094) (end 105.156 113.792) (width 0.25) (layer B.Cu) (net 15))
 (segment (start 105.156 112.1664) (end 107.2261 110.0963) (width 0.25) (layer B.Cu) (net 15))
 (segment (start 105.156 113.792) (end 105.156 112.1664) (width 0.25) (layer B.Cu) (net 15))
 (segment (start 107.2007 124.7567) (end 107.666 125.222) (width 0.25) (layer F.Cu) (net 17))
 (segment (start 106.934 125.222) (end 106.934 123.698) (width 0.25) (layer F.Cu) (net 17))
 (segment (start 108.2756 122.3564) (end 108.2756 122.3391) (width 0.25) (layer F.Cu) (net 17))
 (segment (start 106.934 123.698) (end 108.2756 122.3564) (width 0.25) (layer F.Cu) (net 17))
 (segment (start 105.7008 119.9642) (end 105.41 120.255) (width 0.25) (layer F.Cu) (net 18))
 (segment (start 107.2007 119.9642) (end 105.7008 119.9642) (width 0.25) (layer F.Cu) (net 18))
 (segment (start 105.769199 120.614199) (end 105.41 120.255) (width 0.25) (layer F.Cu) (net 18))
 (segment (start 107.2007 120.614199) (end 105.769199 120.614199) (width 0.25) (layer F.Cu) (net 18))
 (segment (start 105.5692 118.6642) (end 105.41 118.505) (width 0.25) (layer F.Cu) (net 19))
 (segment (start 107.2007 118.6642) (end 105.5692 118.6642) (width 0.25) (layer F.Cu) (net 19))
 (segment (start 106.219201 119.314201) (end 105.41 118.505) (width 0.25) (layer F.Cu) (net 19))
 (segment (start 107.2007 119.314201) (end 106.219201 119.314201) (width 0.25) (layer F.Cu) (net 19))
 (segment (start 113.933 115.57) (end 113.933 114.695) (width 0.25) (layer F.Cu) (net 3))
 (segment (start 113.933 114.695) (end 113.538 114.3) (width 0.25) (layer F.Cu) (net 3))
 (segment (start 109.8436 114.3) (end 108.7387 115.4049) (width 0.25) (layer F.Cu) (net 3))
 (segment (start 113.538 114.3) (end 109.8436 114.3) (width 0.25) (layer F.Cu) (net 3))
 (segment (start 108.2756 115.868) (end 108.2756 117.5893) (width 0.25) (layer F.Cu) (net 3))
 (segment (start 108.7387 115.4049) (end 108.2756 115.868) (width 0.25) (layer F.Cu) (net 3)))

